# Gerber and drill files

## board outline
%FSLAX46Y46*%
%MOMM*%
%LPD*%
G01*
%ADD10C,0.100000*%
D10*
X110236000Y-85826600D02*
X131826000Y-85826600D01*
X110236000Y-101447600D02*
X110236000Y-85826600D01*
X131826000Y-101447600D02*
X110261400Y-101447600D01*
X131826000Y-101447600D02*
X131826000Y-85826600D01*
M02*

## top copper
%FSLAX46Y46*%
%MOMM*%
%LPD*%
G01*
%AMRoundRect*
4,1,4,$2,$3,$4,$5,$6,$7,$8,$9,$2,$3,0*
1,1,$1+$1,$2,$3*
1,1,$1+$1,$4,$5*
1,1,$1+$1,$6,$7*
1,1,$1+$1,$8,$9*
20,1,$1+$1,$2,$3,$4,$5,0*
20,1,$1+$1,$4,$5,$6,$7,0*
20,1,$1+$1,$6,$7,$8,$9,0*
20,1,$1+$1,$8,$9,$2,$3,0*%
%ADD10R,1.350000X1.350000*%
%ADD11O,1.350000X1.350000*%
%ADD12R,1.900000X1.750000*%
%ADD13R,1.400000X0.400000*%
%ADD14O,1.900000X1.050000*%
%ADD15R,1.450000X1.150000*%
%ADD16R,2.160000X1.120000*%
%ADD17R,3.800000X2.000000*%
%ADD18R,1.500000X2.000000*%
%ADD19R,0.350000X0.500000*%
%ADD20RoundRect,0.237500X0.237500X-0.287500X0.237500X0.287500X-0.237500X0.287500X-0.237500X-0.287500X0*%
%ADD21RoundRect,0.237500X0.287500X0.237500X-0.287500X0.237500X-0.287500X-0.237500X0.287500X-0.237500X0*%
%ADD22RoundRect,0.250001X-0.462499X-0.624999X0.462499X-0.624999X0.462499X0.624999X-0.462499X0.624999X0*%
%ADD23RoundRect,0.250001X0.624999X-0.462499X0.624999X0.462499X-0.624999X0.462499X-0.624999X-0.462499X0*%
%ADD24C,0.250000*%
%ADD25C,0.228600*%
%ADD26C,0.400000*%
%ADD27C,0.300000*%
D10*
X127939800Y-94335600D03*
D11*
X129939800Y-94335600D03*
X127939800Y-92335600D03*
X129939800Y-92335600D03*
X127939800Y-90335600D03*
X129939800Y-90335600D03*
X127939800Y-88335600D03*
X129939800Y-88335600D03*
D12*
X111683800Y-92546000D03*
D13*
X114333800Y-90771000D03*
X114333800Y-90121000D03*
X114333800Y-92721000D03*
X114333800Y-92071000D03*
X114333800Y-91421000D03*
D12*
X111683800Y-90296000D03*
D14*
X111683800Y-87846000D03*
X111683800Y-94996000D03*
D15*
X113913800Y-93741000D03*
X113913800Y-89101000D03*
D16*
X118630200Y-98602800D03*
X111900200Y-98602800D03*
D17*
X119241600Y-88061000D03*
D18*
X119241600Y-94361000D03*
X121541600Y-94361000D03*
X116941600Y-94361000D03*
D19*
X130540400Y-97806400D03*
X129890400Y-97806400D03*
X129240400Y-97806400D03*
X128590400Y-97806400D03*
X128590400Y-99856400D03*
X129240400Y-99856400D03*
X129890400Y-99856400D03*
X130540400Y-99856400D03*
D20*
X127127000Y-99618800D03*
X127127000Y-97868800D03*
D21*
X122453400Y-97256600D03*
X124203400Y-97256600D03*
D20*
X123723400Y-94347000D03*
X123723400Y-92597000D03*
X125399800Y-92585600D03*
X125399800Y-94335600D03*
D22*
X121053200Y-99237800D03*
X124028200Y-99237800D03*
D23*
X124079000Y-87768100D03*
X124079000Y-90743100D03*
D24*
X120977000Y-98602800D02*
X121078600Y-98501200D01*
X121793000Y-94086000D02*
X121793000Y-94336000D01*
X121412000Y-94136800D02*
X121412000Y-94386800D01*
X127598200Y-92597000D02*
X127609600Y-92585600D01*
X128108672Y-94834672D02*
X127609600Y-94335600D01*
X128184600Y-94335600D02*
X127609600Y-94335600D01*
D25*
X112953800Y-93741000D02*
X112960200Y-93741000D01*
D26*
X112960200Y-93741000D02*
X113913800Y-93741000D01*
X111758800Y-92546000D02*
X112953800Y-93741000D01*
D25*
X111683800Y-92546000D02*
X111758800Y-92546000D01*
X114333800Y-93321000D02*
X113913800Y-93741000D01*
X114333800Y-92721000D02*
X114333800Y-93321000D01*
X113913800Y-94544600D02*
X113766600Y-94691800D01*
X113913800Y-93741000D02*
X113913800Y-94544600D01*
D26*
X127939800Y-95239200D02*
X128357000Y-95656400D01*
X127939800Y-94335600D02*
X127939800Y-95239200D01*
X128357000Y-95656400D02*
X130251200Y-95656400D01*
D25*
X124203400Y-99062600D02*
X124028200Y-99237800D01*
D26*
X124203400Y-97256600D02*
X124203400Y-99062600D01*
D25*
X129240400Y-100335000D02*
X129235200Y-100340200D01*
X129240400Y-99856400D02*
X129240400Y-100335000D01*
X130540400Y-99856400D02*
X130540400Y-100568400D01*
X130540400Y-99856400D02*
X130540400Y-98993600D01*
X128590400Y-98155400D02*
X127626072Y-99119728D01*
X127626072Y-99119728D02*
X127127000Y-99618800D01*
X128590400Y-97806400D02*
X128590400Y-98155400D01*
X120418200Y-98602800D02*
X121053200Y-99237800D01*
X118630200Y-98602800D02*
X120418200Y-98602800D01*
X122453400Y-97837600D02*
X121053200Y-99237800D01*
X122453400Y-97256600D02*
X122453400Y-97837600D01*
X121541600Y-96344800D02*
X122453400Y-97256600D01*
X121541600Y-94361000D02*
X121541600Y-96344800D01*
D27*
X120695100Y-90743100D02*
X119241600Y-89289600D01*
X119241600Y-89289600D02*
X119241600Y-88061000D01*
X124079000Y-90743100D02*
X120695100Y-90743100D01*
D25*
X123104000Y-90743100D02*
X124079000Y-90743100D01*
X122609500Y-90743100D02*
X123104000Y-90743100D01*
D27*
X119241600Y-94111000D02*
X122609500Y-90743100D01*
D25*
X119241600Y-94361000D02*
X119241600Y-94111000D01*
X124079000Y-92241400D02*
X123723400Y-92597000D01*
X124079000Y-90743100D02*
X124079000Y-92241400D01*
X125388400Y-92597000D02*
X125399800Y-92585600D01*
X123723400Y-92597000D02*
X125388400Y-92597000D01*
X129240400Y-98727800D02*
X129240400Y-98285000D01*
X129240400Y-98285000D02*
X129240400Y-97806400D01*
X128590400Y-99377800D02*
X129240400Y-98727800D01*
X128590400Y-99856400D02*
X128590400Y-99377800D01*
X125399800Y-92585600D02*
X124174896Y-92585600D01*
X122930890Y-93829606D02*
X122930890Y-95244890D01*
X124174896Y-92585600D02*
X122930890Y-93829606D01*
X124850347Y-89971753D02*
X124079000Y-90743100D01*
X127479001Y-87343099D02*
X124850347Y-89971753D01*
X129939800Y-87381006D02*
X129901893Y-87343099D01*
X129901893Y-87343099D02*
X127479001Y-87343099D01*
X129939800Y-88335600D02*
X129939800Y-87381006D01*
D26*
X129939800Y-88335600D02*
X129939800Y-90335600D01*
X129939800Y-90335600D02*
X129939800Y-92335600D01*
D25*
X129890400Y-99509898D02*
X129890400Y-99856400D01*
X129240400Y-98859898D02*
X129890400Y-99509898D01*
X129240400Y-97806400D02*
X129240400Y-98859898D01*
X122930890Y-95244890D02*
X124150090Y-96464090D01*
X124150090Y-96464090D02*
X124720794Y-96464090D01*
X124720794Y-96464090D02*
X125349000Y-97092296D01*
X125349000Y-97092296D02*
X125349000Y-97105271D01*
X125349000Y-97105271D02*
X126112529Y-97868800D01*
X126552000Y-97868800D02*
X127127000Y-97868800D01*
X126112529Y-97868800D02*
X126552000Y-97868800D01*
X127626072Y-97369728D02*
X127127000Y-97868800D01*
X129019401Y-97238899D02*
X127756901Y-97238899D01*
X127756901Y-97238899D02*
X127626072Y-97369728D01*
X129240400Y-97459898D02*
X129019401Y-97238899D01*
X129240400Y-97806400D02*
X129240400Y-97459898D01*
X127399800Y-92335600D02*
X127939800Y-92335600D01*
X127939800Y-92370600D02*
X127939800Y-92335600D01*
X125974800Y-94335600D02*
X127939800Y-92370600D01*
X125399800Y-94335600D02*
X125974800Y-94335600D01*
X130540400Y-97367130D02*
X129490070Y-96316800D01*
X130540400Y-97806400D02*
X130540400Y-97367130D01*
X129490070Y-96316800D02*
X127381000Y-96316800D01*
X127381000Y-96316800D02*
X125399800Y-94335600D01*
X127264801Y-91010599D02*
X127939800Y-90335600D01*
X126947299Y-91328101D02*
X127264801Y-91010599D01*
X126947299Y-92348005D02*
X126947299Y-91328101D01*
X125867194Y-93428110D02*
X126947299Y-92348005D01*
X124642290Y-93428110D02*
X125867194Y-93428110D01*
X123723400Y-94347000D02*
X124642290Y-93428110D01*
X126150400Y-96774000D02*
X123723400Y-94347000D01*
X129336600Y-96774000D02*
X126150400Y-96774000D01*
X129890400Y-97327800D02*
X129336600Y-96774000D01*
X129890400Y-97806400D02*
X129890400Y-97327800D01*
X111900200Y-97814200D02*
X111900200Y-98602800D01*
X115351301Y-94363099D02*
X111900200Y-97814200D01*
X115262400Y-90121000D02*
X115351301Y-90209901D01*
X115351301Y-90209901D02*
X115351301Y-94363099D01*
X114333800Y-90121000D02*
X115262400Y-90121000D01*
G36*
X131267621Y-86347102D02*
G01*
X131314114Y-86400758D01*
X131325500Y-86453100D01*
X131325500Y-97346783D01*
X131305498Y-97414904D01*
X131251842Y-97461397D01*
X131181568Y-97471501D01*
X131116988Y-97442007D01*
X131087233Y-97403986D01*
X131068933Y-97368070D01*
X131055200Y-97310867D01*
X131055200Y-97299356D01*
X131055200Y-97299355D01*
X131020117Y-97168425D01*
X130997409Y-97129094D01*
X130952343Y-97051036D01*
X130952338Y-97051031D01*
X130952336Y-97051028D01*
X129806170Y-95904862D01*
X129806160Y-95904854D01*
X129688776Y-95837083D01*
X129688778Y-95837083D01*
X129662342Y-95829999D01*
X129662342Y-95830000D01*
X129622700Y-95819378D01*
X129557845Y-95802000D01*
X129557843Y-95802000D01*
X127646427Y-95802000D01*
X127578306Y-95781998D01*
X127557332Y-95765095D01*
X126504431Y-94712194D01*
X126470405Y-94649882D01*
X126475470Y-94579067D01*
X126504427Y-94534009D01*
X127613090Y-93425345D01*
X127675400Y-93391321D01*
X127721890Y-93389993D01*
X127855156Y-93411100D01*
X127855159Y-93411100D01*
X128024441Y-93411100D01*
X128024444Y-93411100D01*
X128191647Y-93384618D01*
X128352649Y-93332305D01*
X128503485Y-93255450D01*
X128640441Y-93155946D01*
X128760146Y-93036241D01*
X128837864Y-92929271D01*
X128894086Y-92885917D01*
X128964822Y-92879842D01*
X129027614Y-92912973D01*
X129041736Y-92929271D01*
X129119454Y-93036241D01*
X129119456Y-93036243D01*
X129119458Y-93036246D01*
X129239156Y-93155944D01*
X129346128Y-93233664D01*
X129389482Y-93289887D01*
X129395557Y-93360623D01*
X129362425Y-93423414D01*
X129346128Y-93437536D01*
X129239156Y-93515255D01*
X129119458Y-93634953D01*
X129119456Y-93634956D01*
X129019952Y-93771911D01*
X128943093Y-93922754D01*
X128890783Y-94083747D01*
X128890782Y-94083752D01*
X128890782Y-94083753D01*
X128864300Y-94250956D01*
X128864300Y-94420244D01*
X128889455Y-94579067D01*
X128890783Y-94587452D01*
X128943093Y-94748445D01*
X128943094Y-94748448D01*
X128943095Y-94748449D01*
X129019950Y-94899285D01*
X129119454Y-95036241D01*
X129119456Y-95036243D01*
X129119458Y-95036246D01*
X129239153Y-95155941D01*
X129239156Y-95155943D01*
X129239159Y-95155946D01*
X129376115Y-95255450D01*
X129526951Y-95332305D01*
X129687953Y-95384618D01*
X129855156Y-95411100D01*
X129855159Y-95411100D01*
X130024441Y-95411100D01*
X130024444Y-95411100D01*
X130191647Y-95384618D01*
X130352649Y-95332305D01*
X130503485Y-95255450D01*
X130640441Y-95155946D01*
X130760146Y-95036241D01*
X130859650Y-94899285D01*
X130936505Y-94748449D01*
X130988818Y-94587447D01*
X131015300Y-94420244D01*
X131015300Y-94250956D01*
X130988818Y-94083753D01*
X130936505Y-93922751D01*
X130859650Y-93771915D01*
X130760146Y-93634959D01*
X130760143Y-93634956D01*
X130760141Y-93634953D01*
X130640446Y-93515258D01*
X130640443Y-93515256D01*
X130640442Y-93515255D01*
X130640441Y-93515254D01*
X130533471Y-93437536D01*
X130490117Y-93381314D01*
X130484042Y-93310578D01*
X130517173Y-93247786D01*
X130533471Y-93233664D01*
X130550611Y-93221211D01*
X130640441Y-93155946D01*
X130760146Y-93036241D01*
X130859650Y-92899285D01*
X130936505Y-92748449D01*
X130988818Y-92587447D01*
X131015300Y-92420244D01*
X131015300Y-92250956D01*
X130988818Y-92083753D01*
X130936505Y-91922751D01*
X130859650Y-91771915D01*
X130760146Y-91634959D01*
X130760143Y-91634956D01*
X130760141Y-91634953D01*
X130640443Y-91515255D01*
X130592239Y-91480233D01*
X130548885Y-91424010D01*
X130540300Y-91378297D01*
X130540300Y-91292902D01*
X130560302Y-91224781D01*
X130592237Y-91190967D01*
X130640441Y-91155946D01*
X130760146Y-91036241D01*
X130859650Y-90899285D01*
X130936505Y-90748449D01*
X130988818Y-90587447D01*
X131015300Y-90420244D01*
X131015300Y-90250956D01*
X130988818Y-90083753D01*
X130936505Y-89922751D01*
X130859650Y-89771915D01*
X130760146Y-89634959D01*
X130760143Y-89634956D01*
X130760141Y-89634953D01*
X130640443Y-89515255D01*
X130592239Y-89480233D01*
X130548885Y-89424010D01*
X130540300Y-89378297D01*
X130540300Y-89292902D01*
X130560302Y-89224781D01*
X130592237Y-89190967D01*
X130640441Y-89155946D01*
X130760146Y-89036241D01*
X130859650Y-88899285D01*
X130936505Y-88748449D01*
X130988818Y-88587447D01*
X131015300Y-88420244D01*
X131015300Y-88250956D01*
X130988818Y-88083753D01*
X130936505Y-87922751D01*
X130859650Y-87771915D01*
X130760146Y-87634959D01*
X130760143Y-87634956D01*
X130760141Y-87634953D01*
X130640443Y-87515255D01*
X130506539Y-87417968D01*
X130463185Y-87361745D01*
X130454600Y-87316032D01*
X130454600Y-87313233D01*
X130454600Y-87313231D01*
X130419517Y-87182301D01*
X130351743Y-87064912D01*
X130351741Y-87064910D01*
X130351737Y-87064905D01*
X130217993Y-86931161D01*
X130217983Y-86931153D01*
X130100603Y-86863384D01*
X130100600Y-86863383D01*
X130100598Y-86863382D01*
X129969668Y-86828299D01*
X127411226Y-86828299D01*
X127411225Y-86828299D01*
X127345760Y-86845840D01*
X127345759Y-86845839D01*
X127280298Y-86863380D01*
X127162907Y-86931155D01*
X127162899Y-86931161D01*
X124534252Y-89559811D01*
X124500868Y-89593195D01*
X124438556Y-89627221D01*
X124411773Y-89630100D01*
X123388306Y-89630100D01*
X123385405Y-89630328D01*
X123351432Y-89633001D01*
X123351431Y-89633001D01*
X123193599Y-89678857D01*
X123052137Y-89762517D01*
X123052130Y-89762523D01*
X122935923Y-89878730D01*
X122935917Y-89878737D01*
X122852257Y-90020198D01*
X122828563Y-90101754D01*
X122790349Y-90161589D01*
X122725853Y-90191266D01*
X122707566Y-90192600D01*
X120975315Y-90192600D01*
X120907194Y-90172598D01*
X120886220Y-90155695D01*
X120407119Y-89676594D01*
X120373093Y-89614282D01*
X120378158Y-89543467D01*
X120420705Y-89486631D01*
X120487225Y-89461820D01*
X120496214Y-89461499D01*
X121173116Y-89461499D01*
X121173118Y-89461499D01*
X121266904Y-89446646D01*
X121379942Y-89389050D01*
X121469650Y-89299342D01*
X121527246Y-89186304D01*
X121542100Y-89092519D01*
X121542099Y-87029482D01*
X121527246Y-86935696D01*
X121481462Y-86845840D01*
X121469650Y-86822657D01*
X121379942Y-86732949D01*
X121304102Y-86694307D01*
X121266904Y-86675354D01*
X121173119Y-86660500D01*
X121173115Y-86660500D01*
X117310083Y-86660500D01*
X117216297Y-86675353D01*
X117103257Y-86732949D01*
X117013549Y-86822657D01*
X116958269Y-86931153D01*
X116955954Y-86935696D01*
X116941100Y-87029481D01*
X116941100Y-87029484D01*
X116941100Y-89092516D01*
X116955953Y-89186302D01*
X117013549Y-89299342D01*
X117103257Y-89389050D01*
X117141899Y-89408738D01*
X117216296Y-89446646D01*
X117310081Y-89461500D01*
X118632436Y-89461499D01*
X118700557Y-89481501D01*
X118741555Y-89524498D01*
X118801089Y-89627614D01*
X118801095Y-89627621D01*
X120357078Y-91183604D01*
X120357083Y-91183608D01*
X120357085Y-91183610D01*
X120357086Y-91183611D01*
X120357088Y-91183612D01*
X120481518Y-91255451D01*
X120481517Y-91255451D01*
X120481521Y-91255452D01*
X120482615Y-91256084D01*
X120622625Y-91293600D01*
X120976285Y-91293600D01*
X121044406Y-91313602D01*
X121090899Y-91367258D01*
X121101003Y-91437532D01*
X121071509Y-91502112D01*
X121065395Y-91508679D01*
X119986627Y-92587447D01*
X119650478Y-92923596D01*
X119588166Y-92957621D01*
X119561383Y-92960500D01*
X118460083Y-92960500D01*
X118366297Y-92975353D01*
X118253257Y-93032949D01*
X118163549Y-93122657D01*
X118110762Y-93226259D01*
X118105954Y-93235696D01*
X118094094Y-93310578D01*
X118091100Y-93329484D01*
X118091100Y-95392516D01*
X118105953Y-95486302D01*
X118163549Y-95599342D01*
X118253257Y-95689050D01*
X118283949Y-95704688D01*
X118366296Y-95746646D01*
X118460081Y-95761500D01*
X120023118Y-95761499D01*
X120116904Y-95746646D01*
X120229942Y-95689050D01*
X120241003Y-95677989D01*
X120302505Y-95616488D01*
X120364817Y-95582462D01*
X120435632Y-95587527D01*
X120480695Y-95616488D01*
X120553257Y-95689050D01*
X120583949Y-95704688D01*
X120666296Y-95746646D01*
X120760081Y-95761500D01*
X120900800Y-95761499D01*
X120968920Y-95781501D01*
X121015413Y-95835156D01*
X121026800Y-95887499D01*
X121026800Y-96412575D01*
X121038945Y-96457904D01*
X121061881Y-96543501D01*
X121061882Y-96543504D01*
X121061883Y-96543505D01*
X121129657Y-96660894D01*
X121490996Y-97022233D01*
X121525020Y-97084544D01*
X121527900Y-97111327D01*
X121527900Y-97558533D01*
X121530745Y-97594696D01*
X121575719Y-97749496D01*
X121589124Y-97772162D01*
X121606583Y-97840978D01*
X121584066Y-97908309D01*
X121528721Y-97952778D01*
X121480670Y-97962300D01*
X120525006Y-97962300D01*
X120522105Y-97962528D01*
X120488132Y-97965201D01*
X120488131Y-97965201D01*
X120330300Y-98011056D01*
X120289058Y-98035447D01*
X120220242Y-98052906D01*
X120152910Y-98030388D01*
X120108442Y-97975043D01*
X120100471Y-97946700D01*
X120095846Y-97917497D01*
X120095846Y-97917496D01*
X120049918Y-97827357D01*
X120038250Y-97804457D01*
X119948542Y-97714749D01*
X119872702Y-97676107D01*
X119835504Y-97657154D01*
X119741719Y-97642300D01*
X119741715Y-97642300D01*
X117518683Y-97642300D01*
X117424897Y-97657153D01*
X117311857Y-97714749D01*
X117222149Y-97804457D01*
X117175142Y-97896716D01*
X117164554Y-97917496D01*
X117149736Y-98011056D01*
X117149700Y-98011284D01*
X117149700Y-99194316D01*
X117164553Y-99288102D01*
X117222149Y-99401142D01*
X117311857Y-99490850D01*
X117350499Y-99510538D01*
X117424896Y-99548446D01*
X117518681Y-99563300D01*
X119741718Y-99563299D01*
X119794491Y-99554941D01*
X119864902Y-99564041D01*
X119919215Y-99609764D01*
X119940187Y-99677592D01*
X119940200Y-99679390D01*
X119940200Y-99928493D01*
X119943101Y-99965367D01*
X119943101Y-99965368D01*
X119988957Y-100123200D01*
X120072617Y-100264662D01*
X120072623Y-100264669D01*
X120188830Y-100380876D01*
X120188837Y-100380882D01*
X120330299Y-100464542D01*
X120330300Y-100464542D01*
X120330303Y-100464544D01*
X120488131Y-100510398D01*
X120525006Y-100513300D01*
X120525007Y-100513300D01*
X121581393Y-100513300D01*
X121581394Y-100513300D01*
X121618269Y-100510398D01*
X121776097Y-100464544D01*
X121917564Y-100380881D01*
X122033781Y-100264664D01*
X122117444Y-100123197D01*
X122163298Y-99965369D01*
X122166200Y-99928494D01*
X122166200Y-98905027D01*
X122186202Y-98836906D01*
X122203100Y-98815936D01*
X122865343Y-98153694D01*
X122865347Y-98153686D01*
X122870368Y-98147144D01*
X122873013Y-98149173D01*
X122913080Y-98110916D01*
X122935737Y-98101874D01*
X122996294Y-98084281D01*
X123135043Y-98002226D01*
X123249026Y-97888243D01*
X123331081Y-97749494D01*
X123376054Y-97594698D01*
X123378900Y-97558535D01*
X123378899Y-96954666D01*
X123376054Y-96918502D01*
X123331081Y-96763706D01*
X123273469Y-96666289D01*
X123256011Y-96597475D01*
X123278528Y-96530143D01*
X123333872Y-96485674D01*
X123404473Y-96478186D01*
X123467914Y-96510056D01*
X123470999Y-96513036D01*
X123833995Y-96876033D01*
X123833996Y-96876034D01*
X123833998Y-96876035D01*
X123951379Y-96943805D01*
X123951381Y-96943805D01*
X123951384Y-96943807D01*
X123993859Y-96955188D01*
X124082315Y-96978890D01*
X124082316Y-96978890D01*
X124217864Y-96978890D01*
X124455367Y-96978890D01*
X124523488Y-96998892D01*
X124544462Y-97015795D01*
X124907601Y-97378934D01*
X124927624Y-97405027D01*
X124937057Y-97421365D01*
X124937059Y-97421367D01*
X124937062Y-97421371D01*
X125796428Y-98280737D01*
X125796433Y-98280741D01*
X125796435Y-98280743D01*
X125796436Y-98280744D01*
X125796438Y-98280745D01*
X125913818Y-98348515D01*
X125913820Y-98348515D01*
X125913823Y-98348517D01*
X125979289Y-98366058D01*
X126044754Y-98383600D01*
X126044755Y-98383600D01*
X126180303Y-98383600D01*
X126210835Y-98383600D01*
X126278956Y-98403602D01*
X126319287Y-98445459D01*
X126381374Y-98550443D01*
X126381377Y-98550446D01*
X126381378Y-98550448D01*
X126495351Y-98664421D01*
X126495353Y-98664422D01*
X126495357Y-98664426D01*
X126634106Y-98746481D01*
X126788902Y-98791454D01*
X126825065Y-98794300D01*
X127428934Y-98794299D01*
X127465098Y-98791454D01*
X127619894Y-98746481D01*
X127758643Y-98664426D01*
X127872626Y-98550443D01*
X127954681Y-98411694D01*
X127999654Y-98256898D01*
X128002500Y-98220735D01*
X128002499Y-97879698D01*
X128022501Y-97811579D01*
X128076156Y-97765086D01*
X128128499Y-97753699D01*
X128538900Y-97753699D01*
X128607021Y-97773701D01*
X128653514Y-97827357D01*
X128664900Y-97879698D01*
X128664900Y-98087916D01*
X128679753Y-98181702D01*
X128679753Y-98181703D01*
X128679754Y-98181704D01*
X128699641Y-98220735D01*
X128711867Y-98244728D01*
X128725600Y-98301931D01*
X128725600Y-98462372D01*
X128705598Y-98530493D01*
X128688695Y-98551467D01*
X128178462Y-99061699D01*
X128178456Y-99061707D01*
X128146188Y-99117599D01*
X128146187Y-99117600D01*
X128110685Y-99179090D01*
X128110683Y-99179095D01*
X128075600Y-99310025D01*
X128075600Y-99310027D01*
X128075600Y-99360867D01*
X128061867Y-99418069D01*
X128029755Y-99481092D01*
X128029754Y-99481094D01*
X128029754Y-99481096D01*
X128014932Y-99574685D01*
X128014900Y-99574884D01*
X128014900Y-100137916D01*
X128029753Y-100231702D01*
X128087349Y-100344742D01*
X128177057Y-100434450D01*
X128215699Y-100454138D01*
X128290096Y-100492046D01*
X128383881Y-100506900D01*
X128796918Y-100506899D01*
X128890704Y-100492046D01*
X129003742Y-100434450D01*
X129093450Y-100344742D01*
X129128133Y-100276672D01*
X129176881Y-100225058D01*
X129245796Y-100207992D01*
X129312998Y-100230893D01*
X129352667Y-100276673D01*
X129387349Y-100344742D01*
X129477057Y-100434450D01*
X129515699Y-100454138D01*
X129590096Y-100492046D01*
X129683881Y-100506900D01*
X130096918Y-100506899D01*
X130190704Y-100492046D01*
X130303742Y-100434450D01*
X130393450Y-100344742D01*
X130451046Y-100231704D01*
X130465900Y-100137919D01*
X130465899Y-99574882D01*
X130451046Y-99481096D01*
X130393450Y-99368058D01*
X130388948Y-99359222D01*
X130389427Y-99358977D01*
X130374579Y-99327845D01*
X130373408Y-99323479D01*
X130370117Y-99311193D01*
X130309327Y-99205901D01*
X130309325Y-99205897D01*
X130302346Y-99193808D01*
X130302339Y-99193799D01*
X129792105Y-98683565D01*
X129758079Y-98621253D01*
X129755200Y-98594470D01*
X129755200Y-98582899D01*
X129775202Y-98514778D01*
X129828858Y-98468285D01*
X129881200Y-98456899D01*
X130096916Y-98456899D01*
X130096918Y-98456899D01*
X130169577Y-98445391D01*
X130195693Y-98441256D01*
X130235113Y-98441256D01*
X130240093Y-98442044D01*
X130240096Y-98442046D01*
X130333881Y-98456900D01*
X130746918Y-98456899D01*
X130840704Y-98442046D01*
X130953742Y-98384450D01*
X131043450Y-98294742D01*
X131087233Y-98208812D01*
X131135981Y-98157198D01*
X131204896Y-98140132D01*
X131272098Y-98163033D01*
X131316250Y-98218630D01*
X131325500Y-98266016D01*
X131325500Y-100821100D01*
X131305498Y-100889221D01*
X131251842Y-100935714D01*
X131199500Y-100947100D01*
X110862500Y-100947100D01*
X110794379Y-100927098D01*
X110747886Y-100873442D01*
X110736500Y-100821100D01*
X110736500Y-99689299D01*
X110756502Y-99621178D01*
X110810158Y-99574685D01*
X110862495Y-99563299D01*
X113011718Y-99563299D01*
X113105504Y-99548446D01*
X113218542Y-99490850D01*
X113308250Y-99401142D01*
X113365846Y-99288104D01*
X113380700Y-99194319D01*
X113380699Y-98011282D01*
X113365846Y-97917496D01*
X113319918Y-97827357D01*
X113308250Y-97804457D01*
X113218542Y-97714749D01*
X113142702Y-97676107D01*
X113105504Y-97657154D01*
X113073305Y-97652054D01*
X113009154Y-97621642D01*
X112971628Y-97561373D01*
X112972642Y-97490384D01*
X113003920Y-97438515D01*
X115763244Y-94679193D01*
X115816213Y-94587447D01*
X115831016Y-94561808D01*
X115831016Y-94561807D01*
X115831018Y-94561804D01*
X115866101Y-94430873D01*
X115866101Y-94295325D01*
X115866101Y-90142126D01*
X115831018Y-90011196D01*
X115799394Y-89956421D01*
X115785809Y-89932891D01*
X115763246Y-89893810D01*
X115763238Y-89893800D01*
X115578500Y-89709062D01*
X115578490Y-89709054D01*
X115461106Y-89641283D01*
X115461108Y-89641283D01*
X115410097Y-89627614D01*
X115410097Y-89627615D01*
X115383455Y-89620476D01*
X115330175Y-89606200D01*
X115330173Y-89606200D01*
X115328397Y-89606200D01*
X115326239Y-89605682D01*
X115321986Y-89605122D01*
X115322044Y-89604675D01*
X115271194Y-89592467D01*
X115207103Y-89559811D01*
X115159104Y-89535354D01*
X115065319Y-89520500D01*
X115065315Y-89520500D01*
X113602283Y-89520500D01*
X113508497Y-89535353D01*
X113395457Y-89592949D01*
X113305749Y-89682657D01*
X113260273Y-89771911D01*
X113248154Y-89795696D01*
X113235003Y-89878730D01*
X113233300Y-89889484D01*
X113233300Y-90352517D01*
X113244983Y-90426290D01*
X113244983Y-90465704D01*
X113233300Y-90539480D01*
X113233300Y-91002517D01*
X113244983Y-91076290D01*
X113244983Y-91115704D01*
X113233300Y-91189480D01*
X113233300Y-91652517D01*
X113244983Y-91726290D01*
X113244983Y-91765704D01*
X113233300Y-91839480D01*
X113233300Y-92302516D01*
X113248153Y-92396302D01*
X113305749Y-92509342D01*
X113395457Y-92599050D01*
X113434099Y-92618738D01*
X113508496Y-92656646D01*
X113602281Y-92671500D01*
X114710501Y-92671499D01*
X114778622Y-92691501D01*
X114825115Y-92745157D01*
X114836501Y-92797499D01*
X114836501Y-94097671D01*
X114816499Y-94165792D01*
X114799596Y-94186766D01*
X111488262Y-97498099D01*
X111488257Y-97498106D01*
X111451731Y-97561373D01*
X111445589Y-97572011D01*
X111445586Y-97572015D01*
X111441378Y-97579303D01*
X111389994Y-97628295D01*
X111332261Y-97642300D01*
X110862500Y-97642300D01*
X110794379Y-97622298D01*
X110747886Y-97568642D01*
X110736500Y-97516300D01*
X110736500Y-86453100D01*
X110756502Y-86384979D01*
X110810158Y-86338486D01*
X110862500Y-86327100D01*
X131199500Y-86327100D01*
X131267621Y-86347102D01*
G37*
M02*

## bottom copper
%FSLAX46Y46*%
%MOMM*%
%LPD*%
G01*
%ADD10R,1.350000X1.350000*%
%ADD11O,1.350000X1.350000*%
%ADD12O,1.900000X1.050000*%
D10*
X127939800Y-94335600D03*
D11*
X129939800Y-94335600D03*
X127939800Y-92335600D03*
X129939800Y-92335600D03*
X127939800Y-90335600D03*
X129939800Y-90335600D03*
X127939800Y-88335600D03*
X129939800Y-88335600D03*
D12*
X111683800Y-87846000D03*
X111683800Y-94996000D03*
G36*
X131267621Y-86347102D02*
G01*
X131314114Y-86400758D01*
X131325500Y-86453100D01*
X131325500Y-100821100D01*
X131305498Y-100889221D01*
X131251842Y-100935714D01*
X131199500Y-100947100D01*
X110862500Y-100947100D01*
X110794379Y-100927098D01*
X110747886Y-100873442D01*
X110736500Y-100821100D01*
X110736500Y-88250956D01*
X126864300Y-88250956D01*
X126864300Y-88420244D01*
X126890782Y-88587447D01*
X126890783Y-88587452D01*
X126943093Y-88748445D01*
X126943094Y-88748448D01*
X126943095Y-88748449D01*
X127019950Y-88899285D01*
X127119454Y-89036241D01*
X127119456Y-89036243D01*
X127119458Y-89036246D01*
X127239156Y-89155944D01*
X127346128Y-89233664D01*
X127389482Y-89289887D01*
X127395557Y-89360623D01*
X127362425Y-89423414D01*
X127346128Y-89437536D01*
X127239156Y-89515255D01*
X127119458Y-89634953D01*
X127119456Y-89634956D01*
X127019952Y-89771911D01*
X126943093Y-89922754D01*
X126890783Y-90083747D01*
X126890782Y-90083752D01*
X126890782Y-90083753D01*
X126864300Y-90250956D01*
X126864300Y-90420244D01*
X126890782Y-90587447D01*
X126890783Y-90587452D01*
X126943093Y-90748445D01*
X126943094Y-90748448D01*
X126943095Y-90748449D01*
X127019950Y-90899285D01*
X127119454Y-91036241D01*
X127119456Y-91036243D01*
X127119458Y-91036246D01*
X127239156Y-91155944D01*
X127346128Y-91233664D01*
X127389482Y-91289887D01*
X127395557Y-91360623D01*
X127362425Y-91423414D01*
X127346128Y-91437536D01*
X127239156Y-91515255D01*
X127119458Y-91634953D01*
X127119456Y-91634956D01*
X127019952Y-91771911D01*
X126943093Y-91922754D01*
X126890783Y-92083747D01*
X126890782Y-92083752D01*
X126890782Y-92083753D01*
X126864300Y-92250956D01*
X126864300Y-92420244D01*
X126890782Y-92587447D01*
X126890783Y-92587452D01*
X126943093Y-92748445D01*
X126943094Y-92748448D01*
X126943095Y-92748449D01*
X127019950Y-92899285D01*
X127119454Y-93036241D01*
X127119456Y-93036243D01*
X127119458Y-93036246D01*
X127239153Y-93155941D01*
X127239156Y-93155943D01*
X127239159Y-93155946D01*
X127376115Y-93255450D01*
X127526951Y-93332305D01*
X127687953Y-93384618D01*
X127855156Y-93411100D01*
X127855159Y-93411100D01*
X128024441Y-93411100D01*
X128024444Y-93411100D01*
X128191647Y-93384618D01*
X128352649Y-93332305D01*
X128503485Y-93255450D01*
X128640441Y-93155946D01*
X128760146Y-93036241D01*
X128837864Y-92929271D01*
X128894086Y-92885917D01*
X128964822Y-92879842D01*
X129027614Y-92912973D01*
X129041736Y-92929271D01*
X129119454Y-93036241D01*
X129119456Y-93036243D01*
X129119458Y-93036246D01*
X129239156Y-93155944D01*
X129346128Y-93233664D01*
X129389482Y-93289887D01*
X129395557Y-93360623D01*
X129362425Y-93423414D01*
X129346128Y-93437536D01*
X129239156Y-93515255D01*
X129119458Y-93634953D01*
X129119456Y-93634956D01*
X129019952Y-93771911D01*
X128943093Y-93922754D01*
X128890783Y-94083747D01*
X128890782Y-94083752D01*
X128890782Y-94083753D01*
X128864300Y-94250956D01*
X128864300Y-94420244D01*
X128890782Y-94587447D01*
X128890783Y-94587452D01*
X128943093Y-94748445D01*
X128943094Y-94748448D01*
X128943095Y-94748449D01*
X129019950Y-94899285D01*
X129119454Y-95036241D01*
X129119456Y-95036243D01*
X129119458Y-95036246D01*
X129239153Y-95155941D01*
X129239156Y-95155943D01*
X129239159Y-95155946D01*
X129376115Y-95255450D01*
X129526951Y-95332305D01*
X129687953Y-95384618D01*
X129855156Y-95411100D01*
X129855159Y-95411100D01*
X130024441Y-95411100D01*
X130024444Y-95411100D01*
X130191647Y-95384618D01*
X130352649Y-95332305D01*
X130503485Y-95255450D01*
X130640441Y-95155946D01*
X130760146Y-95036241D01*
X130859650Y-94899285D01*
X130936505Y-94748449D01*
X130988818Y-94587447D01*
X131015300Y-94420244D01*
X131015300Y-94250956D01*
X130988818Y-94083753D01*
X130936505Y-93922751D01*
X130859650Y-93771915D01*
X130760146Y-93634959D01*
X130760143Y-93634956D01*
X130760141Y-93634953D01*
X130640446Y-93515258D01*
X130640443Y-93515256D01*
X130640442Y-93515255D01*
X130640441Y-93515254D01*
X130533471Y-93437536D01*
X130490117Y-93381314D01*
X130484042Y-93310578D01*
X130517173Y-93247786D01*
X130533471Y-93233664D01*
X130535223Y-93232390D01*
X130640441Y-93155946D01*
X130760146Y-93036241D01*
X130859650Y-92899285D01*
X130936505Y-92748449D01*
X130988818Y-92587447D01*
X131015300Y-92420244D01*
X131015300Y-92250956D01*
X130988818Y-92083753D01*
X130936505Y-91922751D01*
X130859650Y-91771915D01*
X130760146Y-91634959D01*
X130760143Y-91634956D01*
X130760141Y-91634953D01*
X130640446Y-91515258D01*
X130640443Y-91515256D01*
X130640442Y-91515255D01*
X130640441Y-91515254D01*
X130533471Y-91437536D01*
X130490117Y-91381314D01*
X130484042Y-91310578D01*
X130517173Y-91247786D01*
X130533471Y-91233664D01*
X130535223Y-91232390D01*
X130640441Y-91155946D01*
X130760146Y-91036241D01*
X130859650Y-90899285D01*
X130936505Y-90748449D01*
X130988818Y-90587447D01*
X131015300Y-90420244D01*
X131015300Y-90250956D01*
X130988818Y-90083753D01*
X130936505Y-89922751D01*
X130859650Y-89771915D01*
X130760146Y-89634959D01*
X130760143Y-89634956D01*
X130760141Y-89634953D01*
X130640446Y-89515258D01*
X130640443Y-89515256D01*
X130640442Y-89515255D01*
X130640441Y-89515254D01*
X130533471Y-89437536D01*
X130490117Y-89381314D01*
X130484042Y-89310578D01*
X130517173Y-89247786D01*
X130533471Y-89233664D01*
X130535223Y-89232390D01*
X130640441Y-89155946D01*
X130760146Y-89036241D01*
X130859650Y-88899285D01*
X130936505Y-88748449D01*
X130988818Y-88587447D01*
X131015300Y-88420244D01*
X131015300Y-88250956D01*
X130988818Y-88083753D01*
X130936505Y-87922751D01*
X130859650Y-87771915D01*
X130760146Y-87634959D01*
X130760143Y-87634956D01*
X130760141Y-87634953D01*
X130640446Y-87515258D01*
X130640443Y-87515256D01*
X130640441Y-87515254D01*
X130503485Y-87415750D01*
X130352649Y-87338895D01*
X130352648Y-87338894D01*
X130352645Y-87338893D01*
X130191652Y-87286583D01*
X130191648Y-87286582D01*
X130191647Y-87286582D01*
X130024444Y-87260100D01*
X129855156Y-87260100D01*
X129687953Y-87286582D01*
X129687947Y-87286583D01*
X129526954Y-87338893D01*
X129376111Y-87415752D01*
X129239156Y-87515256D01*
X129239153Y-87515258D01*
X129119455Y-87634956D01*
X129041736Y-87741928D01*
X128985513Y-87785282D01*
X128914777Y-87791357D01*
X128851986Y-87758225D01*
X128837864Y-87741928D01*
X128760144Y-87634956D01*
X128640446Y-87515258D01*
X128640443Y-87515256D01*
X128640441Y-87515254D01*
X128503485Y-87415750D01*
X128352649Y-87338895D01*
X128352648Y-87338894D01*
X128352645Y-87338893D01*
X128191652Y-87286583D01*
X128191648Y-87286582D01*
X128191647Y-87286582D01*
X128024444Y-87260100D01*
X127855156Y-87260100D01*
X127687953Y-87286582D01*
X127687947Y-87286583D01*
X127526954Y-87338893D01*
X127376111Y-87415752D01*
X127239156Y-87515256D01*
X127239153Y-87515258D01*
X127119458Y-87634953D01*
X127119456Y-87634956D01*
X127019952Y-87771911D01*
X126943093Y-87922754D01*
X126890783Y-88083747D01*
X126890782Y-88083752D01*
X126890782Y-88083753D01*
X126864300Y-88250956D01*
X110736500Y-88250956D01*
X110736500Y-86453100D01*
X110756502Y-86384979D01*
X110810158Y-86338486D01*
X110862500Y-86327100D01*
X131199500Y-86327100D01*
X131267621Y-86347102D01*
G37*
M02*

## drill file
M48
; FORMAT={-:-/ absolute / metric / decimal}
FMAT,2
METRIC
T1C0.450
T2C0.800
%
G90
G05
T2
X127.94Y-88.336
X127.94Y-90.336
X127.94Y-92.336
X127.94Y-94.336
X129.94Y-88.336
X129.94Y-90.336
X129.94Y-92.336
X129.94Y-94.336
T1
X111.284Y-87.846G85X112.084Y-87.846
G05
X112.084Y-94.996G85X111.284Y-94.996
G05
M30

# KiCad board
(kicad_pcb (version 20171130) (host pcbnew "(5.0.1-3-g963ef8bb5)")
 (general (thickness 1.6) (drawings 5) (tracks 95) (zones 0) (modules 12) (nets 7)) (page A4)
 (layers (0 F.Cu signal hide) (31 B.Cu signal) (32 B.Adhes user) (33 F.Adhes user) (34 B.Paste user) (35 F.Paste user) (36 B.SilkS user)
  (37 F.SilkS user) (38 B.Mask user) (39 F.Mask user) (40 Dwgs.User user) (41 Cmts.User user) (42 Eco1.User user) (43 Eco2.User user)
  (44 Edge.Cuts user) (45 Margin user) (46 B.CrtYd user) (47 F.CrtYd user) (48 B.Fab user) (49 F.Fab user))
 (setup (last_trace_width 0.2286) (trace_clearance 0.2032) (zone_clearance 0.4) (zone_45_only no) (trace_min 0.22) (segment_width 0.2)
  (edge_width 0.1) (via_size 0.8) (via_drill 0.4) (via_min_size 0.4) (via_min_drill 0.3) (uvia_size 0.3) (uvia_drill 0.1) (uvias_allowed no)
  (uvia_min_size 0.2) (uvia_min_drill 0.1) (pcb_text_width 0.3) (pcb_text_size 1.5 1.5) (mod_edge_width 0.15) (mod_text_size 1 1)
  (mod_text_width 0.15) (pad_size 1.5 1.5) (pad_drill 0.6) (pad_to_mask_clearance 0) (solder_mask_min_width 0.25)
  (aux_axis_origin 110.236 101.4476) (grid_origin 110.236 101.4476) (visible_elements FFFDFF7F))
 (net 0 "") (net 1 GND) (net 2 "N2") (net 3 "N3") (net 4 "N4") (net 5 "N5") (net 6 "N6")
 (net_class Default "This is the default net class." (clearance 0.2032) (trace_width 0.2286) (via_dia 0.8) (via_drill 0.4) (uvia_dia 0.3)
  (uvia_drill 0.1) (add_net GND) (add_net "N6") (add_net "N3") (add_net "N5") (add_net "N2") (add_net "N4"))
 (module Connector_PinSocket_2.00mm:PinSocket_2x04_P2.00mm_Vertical (layer F.Cu) (at 127.9398 94.3356 180)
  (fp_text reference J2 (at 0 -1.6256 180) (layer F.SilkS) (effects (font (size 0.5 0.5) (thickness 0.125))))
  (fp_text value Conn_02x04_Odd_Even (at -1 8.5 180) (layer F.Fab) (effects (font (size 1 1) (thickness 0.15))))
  (pad 1 thru_hole rect (at 0 0 180) (size 1.35 1.35) (drill 0.8) (layers *.Cu *.Mask) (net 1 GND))
  (pad 2 thru_hole oval (at -2 0 180) (size 1.35 1.35) (drill 0.8) (layers *.Cu *.Mask))
  (pad 3 thru_hole oval (at 0 2 180) (size 1.35 1.35) (drill 0.8) (layers *.Cu *.Mask) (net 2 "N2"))
  (pad 4 thru_hole oval (at -2 2 180) (size 1.35 1.35) (drill 0.8) (layers *.Cu *.Mask) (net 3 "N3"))
  (pad 5 thru_hole oval (at 0 4 180) (size 1.35 1.35) (drill 0.8) (layers *.Cu *.Mask) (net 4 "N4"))
  (pad 6 thru_hole oval (at -2 4 180) (size 1.35 1.35) (drill 0.8) (layers *.Cu *.Mask) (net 3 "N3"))
  (pad 7 thru_hole oval (at 0 6 180) (size 1.35 1.35) (drill 0.8) (layers *.Cu *.Mask))
  (pad 8 thru_hole oval (at -2 6 180) (size 1.35 1.35) (drill 0.8) (layers *.Cu *.Mask) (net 3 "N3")))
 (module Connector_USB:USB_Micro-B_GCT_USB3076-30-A (layer F.Cu) (at 112.8838 91.421 270)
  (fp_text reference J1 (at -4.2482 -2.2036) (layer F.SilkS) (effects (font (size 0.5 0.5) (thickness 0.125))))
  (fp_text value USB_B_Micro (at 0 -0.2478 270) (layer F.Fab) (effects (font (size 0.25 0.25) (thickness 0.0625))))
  (pad 6 smd rect (at 1.125 1.2 270) (size 1.75 1.9) (layers F.Cu F.Paste F.Mask) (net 1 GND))
  (pad 2 smd rect (at -0.65 -1.45 270) (size 0.4 1.4) (layers F.Cu F.Paste F.Mask))
  (pad 1 smd rect (at -1.3 -1.45 270) (size 0.4 1.4) (layers F.Cu F.Paste F.Mask) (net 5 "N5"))
  (pad 5 smd rect (at 1.3 -1.45 270) (size 0.4 1.4) (layers F.Cu F.Paste F.Mask) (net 1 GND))
  (pad 4 smd rect (at 0.65 -1.45 270) (size 0.4 1.4) (layers F.Cu F.Paste F.Mask))
  (pad 3 smd rect (at 0 -1.45 270) (size 0.4 1.4) (layers F.Cu F.Paste F.Mask))
  (pad 6 smd rect (at -1.125 1.2 270) (size 1.75 1.9) (layers F.Cu F.Paste F.Mask) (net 1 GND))
  (pad 6 thru_hole oval (at -3.575 1.2 90) (size 1.05 1.9) (drill oval 0.45 1.25) (layers *.Cu *.Mask) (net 1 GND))
  (pad 6 thru_hole oval (at 3.575 1.2 270) (size 1.05 1.9) (drill oval 0.45 1.25) (layers *.Cu *.Mask) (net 1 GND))
  (pad 6 smd rect (at 2.32 -1.03 270) (size 1.15 1.45) (layers F.Cu F.Paste F.Mask) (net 1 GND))
  (pad 6 smd rect (at -2.32 -1.03 270) (size 1.15 1.45) (layers F.Cu F.Paste F.Mask) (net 1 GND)))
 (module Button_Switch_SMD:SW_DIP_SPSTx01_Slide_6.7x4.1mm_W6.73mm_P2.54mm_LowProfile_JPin (layer F.Cu) (at 115.2652 98.6028)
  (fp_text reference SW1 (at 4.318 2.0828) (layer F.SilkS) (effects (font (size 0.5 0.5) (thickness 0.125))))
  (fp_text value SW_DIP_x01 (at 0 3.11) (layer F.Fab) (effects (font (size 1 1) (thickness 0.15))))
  (pad 2 smd rect (at 3.365 0) (size 2.16 1.12) (layers F.Cu F.Paste F.Mask) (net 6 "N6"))
  (pad 1 smd rect (at -3.365 0) (size 2.16 1.12) (layers F.Cu F.Paste F.Mask) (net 5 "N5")))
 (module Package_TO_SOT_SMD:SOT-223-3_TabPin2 (layer F.Cu) (at 119.2416 91.211 90)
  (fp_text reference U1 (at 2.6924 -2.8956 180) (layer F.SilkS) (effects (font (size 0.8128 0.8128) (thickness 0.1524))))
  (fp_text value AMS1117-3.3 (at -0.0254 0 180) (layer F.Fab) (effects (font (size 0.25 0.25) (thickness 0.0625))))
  (pad 2 smd rect (at 3.15 0 90) (size 2 3.8) (layers F.Cu F.Paste F.Mask) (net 3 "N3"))
  (pad 2 smd rect (at -3.15 0 90) (size 2 1.5) (layers F.Cu F.Paste F.Mask) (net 3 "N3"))
  (pad 3 smd rect (at -3.15 2.3 90) (size 2 1.5) (layers F.Cu F.Paste F.Mask) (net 6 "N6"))
  (pad 1 smd rect (at -3.15 -2.3 90) (size 2 1.5) (layers F.Cu F.Paste F.Mask) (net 1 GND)))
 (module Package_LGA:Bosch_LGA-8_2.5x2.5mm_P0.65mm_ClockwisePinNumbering (layer F.Cu) (at 129.5654 98.8314)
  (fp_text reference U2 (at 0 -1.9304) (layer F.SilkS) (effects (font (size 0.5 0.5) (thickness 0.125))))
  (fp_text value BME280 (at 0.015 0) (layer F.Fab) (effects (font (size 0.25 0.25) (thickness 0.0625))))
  (pad 4 smd rect (at 0.975 -1.025 90) (size 0.5 0.35) (layers F.Cu F.Paste F.Mask) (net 2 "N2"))
  (pad 3 smd rect (at 0.325 -1.025 90) (size 0.5 0.35) (layers F.Cu F.Paste F.Mask) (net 4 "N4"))
  (pad 2 smd rect (at -0.325 -1.025 90) (size 0.5 0.35) (layers F.Cu F.Paste F.Mask) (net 3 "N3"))
  (pad 1 smd rect (at -0.975 -1.025 90) (size 0.5 0.35) (layers F.Cu F.Paste F.Mask) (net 1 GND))
  (pad 8 smd rect (at -0.975 1.025 90) (size 0.5 0.35) (layers F.Cu F.Paste F.Mask) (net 3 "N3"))
  (pad 7 smd rect (at -0.325 1.025 90) (size 0.5 0.35) (layers F.Cu F.Paste F.Mask) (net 1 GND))
  (pad 6 smd rect (at 0.325 1.025 90) (size 0.5 0.35) (layers F.Cu F.Paste F.Mask) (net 3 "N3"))
  (pad 5 smd rect (at 0.975 1.025 90) (size 0.5 0.35) (layers F.Cu F.Paste F.Mask) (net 1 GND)))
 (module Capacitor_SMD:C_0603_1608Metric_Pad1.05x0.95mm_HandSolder (layer F.Cu) (at 127.127 98.7438 90)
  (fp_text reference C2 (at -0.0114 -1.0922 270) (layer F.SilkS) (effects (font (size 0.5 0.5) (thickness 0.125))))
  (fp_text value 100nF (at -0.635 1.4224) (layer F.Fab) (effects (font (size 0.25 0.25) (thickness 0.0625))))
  (pad 1 smd roundrect (at -0.875 0 90) (size 1.05 0.95) (layers F.Cu F.Paste F.Mask) (roundrect_rratio 0.25) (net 1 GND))
  (pad 2 smd roundrect (at 0.875 0 90) (size 1.05 0.95) (layers F.Cu F.Paste F.Mask) (roundrect_rratio 0.25) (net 3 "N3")))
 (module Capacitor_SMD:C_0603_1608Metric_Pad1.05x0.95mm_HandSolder (layer F.Cu) (at 123.3284 97.2566 180)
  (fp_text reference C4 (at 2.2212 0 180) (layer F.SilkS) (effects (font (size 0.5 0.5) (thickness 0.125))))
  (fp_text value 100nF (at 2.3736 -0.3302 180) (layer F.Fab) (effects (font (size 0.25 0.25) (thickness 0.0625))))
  (pad 2 smd roundrect (at 0.875 0 180) (size 1.05 0.95) (layers F.Cu F.Paste F.Mask) (roundrect_rratio 0.25) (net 6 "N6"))
  (pad 1 smd roundrect (at -0.875 0 180) (size 1.05 0.95) (layers F.Cu F.Paste F.Mask) (roundrect_rratio 0.25) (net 1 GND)))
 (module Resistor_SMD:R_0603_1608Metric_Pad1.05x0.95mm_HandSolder (layer F.Cu) (at 123.7234 93.472 90)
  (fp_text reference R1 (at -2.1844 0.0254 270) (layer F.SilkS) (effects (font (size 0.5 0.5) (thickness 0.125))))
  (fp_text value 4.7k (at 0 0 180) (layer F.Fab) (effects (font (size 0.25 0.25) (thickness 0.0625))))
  (pad 1 smd roundrect (at -0.875 0 90) (size 1.05 0.95) (layers F.Cu F.Paste F.Mask) (roundrect_rratio 0.25) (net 4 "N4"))
  (pad 2 smd roundrect (at 0.875 0 90) (size 1.05 0.95) (layers F.Cu F.Paste F.Mask) (roundrect_rratio 0.25) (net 3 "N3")))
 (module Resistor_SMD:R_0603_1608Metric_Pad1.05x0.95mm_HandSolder (layer F.Cu) (at 125.3998 93.4606 90)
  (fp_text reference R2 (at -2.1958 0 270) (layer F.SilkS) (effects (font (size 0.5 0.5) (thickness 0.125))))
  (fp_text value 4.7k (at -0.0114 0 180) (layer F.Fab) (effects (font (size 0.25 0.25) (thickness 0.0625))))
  (pad 2 smd roundrect (at 0.875 0 90) (size 1.05 0.95) (layers F.Cu F.Paste F.Mask) (roundrect_rratio 0.25) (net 3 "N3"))
  (pad 1 smd roundrect (at -0.875 0 90) (size 1.05 0.95) (layers F.Cu F.Paste F.Mask) (roundrect_rratio 0.25) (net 2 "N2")))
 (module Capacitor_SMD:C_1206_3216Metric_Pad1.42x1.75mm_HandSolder (layer F.Cu) (at 122.5407 99.2378)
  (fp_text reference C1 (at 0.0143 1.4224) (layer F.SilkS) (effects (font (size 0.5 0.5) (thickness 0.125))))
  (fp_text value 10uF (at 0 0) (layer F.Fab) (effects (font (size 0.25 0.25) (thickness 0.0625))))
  (pad 1 smd roundrect (at -1.4875 0) (size 1.425 1.75) (layers F.Cu F.Paste F.Mask) (roundrect_rratio 0.175439) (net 6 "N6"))
  (pad 2 smd roundrect (at 1.4875 0) (size 1.425 1.75) (layers F.Cu F.Paste F.Mask) (roundrect_rratio 0.175439) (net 1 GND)))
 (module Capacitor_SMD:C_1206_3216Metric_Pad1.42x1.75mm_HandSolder (layer F.Cu) (at 124.079 89.2556 90)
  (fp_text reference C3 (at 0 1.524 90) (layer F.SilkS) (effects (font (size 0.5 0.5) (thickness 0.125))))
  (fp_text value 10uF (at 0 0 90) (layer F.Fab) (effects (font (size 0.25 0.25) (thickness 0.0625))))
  (pad 2 smd roundrect (at 1.4875 0 90) (size 1.425 1.75) (layers F.Cu F.Paste F.Mask) (roundrect_rratio 0.175439) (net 1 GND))
  (pad 1 smd roundrect (at -1.4875 0 90) (size 1.425 1.75) (layers F.Cu F.Paste F.Mask) (roundrect_rratio 0.175439) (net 3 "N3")))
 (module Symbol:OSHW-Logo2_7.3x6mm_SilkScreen (layer B.Cu) (at 119.507 91.6178 180)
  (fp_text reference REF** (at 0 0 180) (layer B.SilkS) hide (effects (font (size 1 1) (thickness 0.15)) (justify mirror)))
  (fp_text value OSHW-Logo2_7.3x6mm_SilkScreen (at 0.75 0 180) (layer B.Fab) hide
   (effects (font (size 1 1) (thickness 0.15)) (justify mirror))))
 (gr_line (start 110.236 85.8266) (end 131.826 85.8266) (layer Edge.Cuts) (width 0.1))
 (gr_line (start 110.236 101.4476) (end 110.236 85.8266) (layer Edge.Cuts) (width 0.1))
 (gr_line (start 131.826 101.4476) (end 110.2614 101.4476) (layer Edge.Cuts) (width 0.1))
 (gr_line (start 131.826 101.4476) (end 131.826 85.8266) (layer Edge.Cuts) (width 0.1))
 (segment (start 120.977 98.6028) (end 121.0786 98.5012) (width 0.25) (layer F.Cu) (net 6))
 (segment (start 121.793 94.086) (end 121.793 94.336) (width 0.25) (layer F.Cu) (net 6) (status 30))
 (segment (start 121.412 94.1368) (end 121.412 94.3868) (width 0.25) (layer F.Cu) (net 6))
 (segment (start 127.5982 92.597) (end 127.6096 92.5856) (width 0.25) (layer F.Cu) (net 2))
 (segment (start 128.108672 94.834672) (end 127.6096 94.3356) (width 0.25) (layer F.Cu) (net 1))
 (segment (start 128.1846 94.3356) (end 127.6096 94.3356) (width 0.25) (layer F.Cu) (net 1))
 (segment (start 112.9538 93.741) (end 112.9602 93.741) (width 0.2286) (layer F.Cu) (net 1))
 (segment (start 112.9602 93.741) (end 113.9138 93.741) (width 0.4) (layer F.Cu) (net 1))
 (segment (start 111.7588 92.546) (end 112.9538 93.741) (width 0.4) (layer F.Cu) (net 1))
 (segment (start 111.6838 92.546) (end 111.7588 92.546) (width 0.2286) (layer F.Cu) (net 1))
 (segment (start 114.3338 93.321) (end 113.9138 93.741) (width 0.2286) (layer F.Cu) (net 1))
 (segment (start 114.3338 92.721) (end 114.3338 93.321) (width 0.2286) (layer F.Cu) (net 1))
 (segment (start 113.9138 94.5446) (end 113.7666 94.6918) (width 0.2286) (layer F.Cu) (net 1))
 (segment (start 113.9138 93.741) (end 113.9138 94.5446) (width 0.2286) (layer F.Cu) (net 1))
 (segment (start 127.9398 95.2392) (end 128.357 95.6564) (width 0.4) (layer F.Cu) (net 1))
 (segment (start 127.9398 94.3356) (end 127.9398 95.2392) (width 0.4) (layer F.Cu) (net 1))
 (segment (start 128.357 95.6564) (end 130.2512 95.6564) (width 0.4) (layer F.Cu) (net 1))
 (segment (start 124.2034 99.0626) (end 124.0282 99.2378) (width 0.2286) (layer F.Cu) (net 1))
 (segment (start 124.2034 97.2566) (end 124.2034 99.0626) (width 0.4) (layer F.Cu) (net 1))
 (segment (start 129.2404 100.335) (end 129.2352 100.3402) (width 0.2286) (layer F.Cu) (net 1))
 (segment (start 129.2404 99.8564) (end 129.2404 100.335) (width 0.2286) (layer F.Cu) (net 1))
 (segment (start 130.5404 99.8564) (end 130.5404 100.5684) (width 0.2286) (layer F.Cu) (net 1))
 (segment (start 130.5404 99.8564) (end 130.5404 98.9936) (width 0.2286) (layer F.Cu) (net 1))
 (segment (start 128.5904 98.1554) (end 127.626072 99.119728) (width 0.2286) (layer F.Cu) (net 1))
 (segment (start 127.626072 99.119728) (end 127.127 99.6188) (width 0.2286) (layer F.Cu) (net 1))
 (segment (start 128.5904 97.8064) (end 128.5904 98.1554) (width 0.2286) (layer F.Cu) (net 1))
 (segment (start 120.4182 98.6028) (end 121.0532 99.2378) (width 0.2286) (layer F.Cu) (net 6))
 (segment (start 118.6302 98.6028) (end 120.4182 98.6028) (width 0.2286) (layer F.Cu) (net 6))
 (segment (start 122.4534 97.8376) (end 121.0532 99.2378) (width 0.2286) (layer F.Cu) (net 6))
 (segment (start 122.4534 97.2566) (end 122.4534 97.8376) (width 0.2286) (layer F.Cu) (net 6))
 (segment (start 121.5416 96.3448) (end 122.4534 97.2566) (width 0.2286) (layer F.Cu) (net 6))
 (segment (start 121.5416 94.361) (end 121.5416 96.3448) (width 0.2286) (layer F.Cu) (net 6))
 (segment (start 120.6951 90.7431) (end 119.2416 89.2896) (width 0.3) (layer F.Cu) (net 3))
 (segment (start 119.2416 89.2896) (end 119.2416 88.061) (width 0.3) (layer F.Cu) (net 3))
 (segment (start 124.079 90.7431) (end 120.6951 90.7431) (width 0.3) (layer F.Cu) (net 3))
 (segment (start 123.104 90.7431) (end 124.079 90.7431) (width 0.2286) (layer F.Cu) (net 3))
 (segment (start 122.6095 90.7431) (end 123.104 90.7431) (width 0.2286) (layer F.Cu) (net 3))
 (segment (start 119.2416 94.111) (end 122.6095 90.7431) (width 0.3) (layer F.Cu) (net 3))
 (segment (start 119.2416 94.361) (end 119.2416 94.111) (width 0.2286) (layer F.Cu) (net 3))
 (segment (start 124.079 92.2414) (end 123.7234 92.597) (width 0.2286) (layer F.Cu) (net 3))
 (segment (start 124.079 90.7431) (end 124.079 92.2414) (width 0.2286) (layer F.Cu) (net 3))
 (segment (start 125.3884 92.597) (end 125.3998 92.5856) (width 0.2286) (layer F.Cu) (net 3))
 (segment (start 123.7234 92.597) (end 125.3884 92.597) (width 0.2286) (layer F.Cu) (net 3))
 (segment (start 129.2404 98.7278) (end 129.2404 98.285) (width 0.2286) (layer F.Cu) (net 3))
 (segment (start 129.2404 98.285) (end 129.2404 97.8064) (width 0.2286) (layer F.Cu) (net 3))
 (segment (start 128.5904 99.3778) (end 129.2404 98.7278) (width 0.2286) (layer F.Cu) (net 3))
 (segment (start 128.5904 99.8564) (end 128.5904 99.3778) (width 0.2286) (layer F.Cu) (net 3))
 (segment (start 125.3998 92.5856) (end 124.174896 92.5856) (width 0.2286) (layer F.Cu) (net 3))
 (segment (start 122.93089 93.829606) (end 122.93089 95.24489) (width 0.2286) (layer F.Cu) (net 3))
 (segment (start 124.174896 92.5856) (end 122.93089 93.829606) (width 0.2286) (layer F.Cu) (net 3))
 (segment (start 124.850347 89.971753) (end 124.079 90.7431) (width 0.2286) (layer F.Cu) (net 3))
 (segment (start 127.479001 87.343099) (end 124.850347 89.971753) (width 0.2286) (layer F.Cu) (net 3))
 (segment (start 129.9398 87.381006) (end 129.901893 87.343099) (width 0.2286) (layer F.Cu) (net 3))
 (segment (start 129.901893 87.343099) (end 127.479001 87.343099) (width 0.2286) (layer F.Cu) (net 3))
 (segment (start 129.9398 88.3356) (end 129.9398 87.381006) (width 0.2286) (layer F.Cu) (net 3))
 (segment (start 129.9398 88.3356) (end 129.9398 90.3356) (width 0.4) (layer F.Cu) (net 3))
 (segment (start 129.9398 90.3356) (end 129.9398 92.3356) (width 0.4) (layer F.Cu) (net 3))
 (segment (start 129.8904 99.509898) (end 129.8904 99.8564) (width 0.2286) (layer F.Cu) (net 3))
 (segment (start 129.2404 98.859898) (end 129.8904 99.509898) (width 0.2286) (layer F.Cu) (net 3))
 (segment (start 129.2404 97.8064) (end 129.2404 98.859898) (width 0.2286) (layer F.Cu) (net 3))
 (segment (start 122.93089 95.24489) (end 124.15009 96.46409) (width 0.2286) (layer F.Cu) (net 3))
 (segment (start 124.15009 96.46409) (end 124.720794 96.46409) (width 0.2286) (layer F.Cu) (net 3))
 (segment (start 124.720794 96.46409) (end 125.349 97.092296) (width 0.2286) (layer F.Cu) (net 3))
 (segment (start 125.349 97.092296) (end 125.349 97.105271) (width 0.2286) (layer F.Cu) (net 3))
 (segment (start 125.349 97.105271) (end 126.112529 97.8688) (width 0.2286) (layer F.Cu) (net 3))
 (segment (start 126.552 97.8688) (end 127.127 97.8688) (width 0.2286) (layer F.Cu) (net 3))
 (segment (start 126.112529 97.8688) (end 126.552 97.8688) (width 0.2286) (layer F.Cu) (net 3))
 (segment (start 127.626072 97.369728) (end 127.127 97.8688) (width 0.2286) (layer F.Cu) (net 3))
 (segment (start 129.019401 97.238899) (end 127.756901 97.238899) (width 0.2286) (layer F.Cu) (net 3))
 (segment (start 127.756901 97.238899) (end 127.626072 97.369728) (width 0.2286) (layer F.Cu) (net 3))
 (segment (start 129.2404 97.459898) (end 129.019401 97.238899) (width 0.2286) (layer F.Cu) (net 3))
 (segment (start 129.2404 97.8064) (end 129.2404 97.459898) (width 0.2286) (layer F.Cu) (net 3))
 (segment (start 127.3998 92.3356) (end 127.9398 92.3356) (width 0.2286) (layer F.Cu) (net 2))
 (segment (start 127.9398 92.3706) (end 127.9398 92.3356) (width 0.2286) (layer F.Cu) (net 2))
 (segment (start 125.9748 94.3356) (end 127.9398 92.3706) (width 0.2286) (layer F.Cu) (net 2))
 (segment (start 125.3998 94.3356) (end 125.9748 94.3356) (width 0.2286) (layer F.Cu) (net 2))
 (segment (start 130.5404 97.36713) (end 129.49007 96.3168) (width 0.2286) (layer F.Cu) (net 2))
 (segment (start 130.5404 97.8064) (end 130.5404 97.36713) (width 0.2286) (layer F.Cu) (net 2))
 (segment (start 129.49007 96.3168) (end 127.381 96.3168) (width 0.2286) (layer F.Cu) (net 2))
 (segment (start 127.381 96.3168) (end 125.3998 94.3356) (width 0.2286) (layer F.Cu) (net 2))
 (segment (start 127.264801 91.010599) (end 127.9398 90.3356) (width 0.2286) (layer F.Cu) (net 4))
 (segment (start 126.947299 91.328101) (end 127.264801 91.010599) (width 0.2286) (layer F.Cu) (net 4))
 (segment (start 126.947299 92.348005) (end 126.947299 91.328101) (width 0.2286) (layer F.Cu) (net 4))
 (segment (start 125.867194 93.42811) (end 126.947299 92.348005) (width 0.2286) (layer F.Cu) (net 4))
 (segment (start 124.64229 93.42811) (end 125.867194 93.42811) (width 0.2286) (layer F.Cu) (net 4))
 (segment (start 123.7234 94.347) (end 124.64229 93.42811) (width 0.2286) (layer F.Cu) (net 4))
 (segment (start 126.1504 96.774) (end 123.7234 94.347) (width 0.2286) (layer F.Cu) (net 4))
 (segment (start 129.3366 96.774) (end 126.1504 96.774) (width 0.2286) (layer F.Cu) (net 4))
 (segment (start 129.8904 97.3278) (end 129.3366 96.774) (width 0.2286) (layer F.Cu) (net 4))
 (segment (start 129.8904 97.8064) (end 129.8904 97.3278) (width 0.2286) (layer F.Cu) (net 4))
 (segment (start 111.9002 97.8142) (end 111.9002 98.6028) (width 0.2286) (layer F.Cu) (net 5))
 (segment (start 115.351301 94.363099) (end 111.9002 97.8142) (width 0.2286) (layer F.Cu) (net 5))
 (segment (start 115.2624 90.121) (end 115.351301 90.209901) (width 0.2286) (layer F.Cu) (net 5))
 (segment (start 115.351301 90.209901) (end 115.351301 94.363099) (width 0.2286) (layer F.Cu) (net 5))
 (segment (start 114.3338 90.121) (end 115.2624 90.121) (width 0.2286) (layer F.Cu) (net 5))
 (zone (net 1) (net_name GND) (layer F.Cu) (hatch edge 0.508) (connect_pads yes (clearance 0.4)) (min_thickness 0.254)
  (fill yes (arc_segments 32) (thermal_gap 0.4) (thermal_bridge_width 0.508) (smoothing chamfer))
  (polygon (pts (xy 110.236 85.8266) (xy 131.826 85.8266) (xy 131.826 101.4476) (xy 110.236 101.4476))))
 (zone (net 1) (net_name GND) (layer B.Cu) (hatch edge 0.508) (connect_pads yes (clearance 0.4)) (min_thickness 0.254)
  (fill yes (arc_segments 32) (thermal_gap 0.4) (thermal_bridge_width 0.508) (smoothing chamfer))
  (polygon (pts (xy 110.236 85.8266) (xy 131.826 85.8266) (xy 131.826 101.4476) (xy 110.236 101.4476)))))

